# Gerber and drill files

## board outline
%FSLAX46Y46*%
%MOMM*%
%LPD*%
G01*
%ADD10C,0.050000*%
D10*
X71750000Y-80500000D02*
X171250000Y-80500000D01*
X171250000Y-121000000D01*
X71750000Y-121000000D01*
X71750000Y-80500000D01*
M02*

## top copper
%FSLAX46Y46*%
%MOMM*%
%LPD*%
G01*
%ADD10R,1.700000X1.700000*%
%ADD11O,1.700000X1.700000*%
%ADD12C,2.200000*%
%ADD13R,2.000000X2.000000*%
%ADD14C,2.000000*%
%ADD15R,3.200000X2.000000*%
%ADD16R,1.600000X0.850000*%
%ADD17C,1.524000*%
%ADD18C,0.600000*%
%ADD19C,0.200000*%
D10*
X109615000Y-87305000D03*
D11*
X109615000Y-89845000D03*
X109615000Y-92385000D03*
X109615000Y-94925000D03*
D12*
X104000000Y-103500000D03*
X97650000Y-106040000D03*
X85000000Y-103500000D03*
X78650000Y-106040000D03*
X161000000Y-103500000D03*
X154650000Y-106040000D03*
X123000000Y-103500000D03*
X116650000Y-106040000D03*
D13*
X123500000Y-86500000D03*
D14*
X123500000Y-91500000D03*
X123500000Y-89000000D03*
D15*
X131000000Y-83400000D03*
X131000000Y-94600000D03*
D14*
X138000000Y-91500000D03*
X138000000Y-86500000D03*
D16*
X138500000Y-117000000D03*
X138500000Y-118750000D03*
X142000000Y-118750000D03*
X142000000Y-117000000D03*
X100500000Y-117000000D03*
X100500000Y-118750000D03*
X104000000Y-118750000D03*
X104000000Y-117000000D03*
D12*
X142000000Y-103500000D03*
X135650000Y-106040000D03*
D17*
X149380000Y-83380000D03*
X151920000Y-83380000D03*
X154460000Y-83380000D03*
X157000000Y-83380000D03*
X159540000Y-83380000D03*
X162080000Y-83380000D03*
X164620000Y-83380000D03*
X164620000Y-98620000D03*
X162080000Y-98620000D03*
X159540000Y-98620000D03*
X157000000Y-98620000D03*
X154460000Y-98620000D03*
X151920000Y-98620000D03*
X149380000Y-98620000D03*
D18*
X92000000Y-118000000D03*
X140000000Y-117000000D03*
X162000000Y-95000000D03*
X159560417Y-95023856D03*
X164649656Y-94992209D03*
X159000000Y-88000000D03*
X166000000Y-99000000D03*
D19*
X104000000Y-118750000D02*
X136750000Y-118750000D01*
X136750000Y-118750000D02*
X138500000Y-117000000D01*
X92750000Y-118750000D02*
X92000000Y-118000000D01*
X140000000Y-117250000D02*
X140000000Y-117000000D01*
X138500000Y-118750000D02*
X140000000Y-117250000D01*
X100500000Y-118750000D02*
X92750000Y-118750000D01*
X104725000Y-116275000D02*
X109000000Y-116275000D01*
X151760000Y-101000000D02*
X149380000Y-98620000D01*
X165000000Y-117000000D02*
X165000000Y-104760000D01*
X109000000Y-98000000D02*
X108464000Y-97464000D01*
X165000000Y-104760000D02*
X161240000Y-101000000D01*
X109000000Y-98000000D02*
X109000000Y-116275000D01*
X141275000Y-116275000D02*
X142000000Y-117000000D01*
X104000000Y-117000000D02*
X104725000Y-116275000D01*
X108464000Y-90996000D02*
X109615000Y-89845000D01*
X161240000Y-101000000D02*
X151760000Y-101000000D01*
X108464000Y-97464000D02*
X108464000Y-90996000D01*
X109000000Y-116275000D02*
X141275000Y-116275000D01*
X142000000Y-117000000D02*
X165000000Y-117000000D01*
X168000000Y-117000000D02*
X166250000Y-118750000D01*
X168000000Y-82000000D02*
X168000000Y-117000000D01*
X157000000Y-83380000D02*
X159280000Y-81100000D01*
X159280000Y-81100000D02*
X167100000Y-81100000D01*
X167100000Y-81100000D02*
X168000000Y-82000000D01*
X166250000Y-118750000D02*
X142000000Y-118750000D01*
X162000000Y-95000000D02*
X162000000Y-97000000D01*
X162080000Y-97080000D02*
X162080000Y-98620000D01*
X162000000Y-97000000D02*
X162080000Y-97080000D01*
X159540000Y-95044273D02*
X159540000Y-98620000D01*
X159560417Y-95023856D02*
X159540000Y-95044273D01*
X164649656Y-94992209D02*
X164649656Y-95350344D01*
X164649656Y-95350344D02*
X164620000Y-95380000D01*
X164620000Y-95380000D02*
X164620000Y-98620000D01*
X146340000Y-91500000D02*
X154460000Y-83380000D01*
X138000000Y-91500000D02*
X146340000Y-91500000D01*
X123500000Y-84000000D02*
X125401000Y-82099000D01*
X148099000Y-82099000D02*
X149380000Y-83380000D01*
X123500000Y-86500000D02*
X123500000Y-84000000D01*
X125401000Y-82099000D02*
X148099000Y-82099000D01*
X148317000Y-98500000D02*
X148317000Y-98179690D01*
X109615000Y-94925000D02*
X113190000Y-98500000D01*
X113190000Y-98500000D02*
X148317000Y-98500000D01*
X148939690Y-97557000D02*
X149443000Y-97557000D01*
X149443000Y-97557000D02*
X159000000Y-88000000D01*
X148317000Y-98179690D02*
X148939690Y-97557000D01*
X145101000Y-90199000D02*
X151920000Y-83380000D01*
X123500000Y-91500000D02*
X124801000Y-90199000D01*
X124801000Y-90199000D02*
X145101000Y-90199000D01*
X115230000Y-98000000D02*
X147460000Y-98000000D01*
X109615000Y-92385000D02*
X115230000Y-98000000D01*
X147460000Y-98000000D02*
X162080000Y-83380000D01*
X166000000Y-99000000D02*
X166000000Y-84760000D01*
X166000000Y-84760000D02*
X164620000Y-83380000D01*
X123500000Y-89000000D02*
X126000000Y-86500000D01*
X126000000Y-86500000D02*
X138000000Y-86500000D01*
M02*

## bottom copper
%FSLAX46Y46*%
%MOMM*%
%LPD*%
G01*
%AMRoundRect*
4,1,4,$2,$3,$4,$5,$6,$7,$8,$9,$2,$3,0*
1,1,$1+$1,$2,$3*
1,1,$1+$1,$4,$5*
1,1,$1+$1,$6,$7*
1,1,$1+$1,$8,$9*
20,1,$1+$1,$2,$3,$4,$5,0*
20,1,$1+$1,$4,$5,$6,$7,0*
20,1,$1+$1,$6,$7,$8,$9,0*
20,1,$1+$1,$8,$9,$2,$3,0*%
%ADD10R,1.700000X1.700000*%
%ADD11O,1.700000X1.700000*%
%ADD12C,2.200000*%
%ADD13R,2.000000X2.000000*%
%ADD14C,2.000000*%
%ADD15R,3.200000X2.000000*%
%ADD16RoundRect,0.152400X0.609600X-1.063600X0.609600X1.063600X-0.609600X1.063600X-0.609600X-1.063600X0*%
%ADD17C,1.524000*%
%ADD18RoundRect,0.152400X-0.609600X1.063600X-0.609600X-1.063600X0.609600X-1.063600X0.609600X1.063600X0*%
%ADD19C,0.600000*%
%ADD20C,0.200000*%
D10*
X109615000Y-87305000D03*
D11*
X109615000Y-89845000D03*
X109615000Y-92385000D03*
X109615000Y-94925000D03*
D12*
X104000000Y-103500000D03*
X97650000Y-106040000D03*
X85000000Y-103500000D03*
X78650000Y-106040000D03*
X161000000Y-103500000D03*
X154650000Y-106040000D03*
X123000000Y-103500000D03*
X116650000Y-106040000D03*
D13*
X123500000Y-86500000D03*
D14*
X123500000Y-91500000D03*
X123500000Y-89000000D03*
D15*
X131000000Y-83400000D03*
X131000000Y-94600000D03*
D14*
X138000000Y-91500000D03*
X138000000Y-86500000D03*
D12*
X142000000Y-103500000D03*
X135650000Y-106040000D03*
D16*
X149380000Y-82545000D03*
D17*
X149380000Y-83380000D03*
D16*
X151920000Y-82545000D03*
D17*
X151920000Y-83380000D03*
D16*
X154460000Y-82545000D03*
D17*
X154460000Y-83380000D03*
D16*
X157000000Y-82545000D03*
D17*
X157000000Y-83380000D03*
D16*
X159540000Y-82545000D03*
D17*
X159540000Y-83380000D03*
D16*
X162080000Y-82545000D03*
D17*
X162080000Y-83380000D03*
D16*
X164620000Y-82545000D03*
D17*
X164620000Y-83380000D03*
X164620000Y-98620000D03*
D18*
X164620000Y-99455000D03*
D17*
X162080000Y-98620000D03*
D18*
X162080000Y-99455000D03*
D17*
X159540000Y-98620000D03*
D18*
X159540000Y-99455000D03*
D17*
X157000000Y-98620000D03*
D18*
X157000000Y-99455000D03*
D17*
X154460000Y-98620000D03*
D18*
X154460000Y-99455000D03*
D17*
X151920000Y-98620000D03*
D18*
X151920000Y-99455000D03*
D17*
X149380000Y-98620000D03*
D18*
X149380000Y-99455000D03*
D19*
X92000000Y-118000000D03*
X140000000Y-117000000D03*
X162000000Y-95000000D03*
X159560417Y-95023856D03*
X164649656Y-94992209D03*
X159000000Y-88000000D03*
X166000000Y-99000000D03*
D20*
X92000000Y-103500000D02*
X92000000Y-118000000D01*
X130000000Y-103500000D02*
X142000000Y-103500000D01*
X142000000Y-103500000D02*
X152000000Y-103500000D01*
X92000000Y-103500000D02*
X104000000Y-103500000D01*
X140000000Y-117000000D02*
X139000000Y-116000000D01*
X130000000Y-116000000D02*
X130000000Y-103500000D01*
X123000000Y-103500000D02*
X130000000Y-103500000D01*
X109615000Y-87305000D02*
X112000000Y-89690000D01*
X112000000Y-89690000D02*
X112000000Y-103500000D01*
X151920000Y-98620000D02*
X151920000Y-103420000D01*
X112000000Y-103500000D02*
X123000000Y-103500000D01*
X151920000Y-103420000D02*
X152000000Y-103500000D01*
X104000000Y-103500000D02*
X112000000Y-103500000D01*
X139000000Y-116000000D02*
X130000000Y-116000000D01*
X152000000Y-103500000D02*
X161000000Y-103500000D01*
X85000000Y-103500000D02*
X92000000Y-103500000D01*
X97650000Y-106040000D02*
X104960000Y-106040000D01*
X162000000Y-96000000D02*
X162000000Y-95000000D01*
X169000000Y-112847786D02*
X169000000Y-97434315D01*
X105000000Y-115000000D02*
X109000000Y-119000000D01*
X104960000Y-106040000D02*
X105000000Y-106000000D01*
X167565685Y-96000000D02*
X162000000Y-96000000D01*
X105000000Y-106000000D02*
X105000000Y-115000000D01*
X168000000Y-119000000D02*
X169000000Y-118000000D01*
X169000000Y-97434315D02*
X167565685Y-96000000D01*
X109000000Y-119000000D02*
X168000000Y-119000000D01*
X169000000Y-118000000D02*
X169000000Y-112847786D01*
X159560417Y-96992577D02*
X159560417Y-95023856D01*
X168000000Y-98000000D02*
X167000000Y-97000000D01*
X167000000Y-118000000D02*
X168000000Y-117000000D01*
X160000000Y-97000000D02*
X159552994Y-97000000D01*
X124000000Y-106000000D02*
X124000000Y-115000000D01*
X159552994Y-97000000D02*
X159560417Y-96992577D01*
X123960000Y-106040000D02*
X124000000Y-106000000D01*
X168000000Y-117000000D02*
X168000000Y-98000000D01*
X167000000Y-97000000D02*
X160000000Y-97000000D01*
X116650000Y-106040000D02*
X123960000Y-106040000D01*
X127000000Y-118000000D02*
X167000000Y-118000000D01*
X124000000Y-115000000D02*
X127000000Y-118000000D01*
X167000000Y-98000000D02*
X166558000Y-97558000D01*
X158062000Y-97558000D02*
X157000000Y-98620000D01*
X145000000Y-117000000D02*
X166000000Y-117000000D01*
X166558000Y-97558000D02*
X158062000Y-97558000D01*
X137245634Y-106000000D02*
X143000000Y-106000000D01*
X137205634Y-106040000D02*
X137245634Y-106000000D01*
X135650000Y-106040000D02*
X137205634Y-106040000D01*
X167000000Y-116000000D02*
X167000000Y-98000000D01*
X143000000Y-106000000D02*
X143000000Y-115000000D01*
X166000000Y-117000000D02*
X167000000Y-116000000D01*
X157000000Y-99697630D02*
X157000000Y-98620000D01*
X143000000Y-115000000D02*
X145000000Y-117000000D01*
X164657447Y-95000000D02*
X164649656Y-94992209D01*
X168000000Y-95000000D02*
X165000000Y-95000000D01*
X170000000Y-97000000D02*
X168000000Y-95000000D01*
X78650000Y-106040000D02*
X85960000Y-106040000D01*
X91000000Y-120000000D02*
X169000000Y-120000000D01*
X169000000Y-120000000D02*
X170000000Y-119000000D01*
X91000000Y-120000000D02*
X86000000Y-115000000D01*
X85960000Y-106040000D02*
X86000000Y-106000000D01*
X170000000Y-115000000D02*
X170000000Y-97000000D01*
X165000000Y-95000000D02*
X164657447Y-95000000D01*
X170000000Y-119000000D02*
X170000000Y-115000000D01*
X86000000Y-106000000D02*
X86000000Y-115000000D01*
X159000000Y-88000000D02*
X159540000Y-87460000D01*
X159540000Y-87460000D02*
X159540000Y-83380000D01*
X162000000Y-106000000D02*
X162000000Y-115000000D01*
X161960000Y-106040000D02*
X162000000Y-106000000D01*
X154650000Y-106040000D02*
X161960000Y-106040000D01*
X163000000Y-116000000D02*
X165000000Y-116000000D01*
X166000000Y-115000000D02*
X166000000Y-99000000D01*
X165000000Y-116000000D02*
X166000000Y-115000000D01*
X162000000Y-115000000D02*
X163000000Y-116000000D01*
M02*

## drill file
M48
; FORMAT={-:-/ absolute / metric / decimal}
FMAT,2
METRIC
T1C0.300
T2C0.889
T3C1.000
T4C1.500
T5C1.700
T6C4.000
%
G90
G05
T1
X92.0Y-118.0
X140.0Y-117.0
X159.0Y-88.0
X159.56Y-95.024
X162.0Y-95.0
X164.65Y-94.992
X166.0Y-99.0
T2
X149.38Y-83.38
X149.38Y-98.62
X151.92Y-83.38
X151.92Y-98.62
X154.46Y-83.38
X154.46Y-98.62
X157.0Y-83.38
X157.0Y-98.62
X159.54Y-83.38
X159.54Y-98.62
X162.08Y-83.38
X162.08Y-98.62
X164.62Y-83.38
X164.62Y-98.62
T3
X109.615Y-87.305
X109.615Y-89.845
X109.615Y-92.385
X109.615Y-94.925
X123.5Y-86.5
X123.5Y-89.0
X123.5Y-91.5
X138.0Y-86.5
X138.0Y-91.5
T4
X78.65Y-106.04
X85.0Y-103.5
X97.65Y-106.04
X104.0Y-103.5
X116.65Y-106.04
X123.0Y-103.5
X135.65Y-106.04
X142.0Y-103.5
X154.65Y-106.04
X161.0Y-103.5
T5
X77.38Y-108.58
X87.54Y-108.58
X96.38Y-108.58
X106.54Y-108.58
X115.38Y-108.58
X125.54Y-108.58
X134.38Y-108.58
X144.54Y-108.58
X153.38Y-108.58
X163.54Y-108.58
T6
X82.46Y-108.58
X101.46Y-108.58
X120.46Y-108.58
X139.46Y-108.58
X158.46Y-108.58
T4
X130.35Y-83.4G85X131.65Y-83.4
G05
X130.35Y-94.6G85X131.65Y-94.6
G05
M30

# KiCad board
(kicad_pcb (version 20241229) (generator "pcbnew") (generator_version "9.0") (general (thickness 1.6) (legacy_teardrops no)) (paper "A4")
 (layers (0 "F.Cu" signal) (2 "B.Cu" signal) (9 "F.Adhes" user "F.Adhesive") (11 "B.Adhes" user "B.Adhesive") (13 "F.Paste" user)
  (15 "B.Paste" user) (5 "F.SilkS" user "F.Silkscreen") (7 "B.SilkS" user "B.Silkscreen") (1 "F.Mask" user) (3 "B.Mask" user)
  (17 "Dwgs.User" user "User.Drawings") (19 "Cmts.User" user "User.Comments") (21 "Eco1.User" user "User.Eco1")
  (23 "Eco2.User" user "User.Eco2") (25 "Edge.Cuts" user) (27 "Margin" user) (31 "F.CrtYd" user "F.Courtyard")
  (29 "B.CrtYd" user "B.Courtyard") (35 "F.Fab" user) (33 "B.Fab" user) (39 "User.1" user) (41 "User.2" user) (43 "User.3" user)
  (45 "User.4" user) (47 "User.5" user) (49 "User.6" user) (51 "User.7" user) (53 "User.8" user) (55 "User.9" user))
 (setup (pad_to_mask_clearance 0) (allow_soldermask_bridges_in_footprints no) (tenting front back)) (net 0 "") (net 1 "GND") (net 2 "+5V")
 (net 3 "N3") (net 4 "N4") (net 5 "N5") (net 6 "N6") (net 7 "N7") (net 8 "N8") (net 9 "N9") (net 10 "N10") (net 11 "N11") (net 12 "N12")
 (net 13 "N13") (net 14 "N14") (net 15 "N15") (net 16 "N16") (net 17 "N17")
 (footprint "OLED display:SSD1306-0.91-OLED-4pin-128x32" (layer "F.Cu") (at 73.115 85.115)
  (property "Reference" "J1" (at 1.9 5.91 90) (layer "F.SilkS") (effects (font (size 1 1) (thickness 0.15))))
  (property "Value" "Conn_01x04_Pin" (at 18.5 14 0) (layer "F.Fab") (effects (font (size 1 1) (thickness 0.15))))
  (pad "1" thru_hole rect (at 36.5 2.19) (size 1.7 1.7) (drill 1) (layers "*.Cu" "*.Mask") (remove_unused_layers no) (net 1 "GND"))
  (pad "2" thru_hole oval (at 36.5 4.73) (size 1.7 1.7) (drill 1) (layers "*.Cu" "*.Mask") (remove_unused_layers no) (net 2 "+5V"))
  (pad "3" thru_hole oval (at 36.5 7.27) (size 1.7 1.7) (drill 1) (layers "*.Cu" "*.Mask") (remove_unused_layers no) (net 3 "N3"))
  (pad "4" thru_hole oval (at 36.5 9.81) (size 1.7 1.7) (drill 1) (layers "*.Cu" "*.Mask") (remove_unused_layers no) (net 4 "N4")))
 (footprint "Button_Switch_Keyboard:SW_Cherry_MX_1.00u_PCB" (layer "F.Cu") (at 104 103.5)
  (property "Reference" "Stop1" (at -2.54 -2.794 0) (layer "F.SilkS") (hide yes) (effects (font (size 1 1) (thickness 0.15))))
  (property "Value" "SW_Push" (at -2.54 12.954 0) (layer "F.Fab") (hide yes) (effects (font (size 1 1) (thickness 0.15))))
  (pad "" np_thru_hole circle (at -7.62 5.08) (size 1.7 1.7) (drill 1.7) (layers "*.Cu" "*.Mask"))
  (pad "" np_thru_hole circle (at -2.54 5.08) (size 4 4) (drill 4) (layers "*.Cu" "*.Mask"))
  (pad "" np_thru_hole circle (at 2.54 5.08) (size 1.7 1.7) (drill 1.7) (layers "*.Cu" "*.Mask"))
  (pad "1" thru_hole circle (at 0 0) (size 2.2 2.2) (drill 1.5) (layers "*.Cu" "*.Mask") (remove_unused_layers no) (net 1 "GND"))
  (pad "2" thru_hole circle (at -6.35 2.54) (size 2.2 2.2) (drill 1.5) (layers "*.Cu" "*.Mask") (remove_unused_layers no) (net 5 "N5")))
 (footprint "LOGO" (layer "F.Cu") (at 120 108.58)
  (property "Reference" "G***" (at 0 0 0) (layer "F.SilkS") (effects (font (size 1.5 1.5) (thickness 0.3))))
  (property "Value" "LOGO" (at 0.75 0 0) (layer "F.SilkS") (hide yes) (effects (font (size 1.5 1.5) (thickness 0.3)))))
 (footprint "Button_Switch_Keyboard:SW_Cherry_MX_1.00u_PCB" (layer "F.Cu") (at 85 103.5)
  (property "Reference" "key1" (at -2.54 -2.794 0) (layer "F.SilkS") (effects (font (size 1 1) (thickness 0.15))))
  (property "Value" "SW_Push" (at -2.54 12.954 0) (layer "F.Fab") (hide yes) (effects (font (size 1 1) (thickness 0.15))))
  (pad "" np_thru_hole circle (at -7.62 5.08) (size 1.7 1.7) (drill 1.7) (layers "*.Cu" "*.Mask"))
  (pad "" np_thru_hole circle (at -2.54 5.08) (size 4 4) (drill 4) (layers "*.Cu" "*.Mask"))
  (pad "" np_thru_hole circle (at 2.54 5.08) (size 1.7 1.7) (drill 1.7) (layers "*.Cu" "*.Mask"))
  (pad "1" thru_hole circle (at 0 0) (size 2.2 2.2) (drill 1.5) (layers "*.Cu" "*.Mask") (remove_unused_layers no) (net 1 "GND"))
  (pad "2" thru_hole circle (at -6.35 2.54) (size 2.2 2.2) (drill 1.5) (layers "*.Cu" "*.Mask") (remove_unused_layers no) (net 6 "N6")))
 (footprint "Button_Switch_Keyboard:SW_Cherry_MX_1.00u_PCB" (layer "F.Cu") (at 161 103.5)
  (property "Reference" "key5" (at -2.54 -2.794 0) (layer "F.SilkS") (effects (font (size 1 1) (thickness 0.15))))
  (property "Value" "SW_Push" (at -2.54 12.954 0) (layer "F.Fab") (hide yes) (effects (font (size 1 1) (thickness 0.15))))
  (pad "" np_thru_hole circle (at -7.62 5.08) (size 1.7 1.7) (drill 1.7) (layers "*.Cu" "*.Mask"))
  (pad "" np_thru_hole circle (at -2.54 5.08) (size 4 4) (drill 4) (layers "*.Cu" "*.Mask"))
  (pad "" np_thru_hole circle (at 2.54 5.08) (size 1.7 1.7) (drill 1.7) (layers "*.Cu" "*.Mask"))
  (pad "1" thru_hole circle (at 0 0) (size 2.2 2.2) (drill 1.5) (layers "*.Cu" "*.Mask") (remove_unused_layers no) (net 1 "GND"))
  (pad "2" thru_hole circle (at -6.35 2.54) (size 2.2 2.2) (drill 1.5) (layers "*.Cu" "*.Mask") (remove_unused_layers no) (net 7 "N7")))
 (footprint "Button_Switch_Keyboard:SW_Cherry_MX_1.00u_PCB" (layer "F.Cu") (at 123 103.5)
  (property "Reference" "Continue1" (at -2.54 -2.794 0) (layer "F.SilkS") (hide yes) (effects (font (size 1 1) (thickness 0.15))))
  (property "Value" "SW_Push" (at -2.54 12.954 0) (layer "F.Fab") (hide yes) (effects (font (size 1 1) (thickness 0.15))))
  (pad "" np_thru_hole circle (at -7.62 5.08) (size 1.7 1.7) (drill 1.7) (layers "*.Cu" "*.Mask"))
  (pad "" np_thru_hole circle (at -2.54 5.08) (size 4 4) (drill 4) (layers "*.Cu" "*.Mask"))
  (pad "" np_thru_hole circle (at 2.54 5.08) (size 1.7 1.7) (drill 1.7) (layers "*.Cu" "*.Mask"))
  (pad "1" thru_hole circle (at 0 0) (size 2.2 2.2) (drill 1.5) (layers "*.Cu" "*.Mask") (remove_unused_layers no) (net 1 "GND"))
  (pad "2" thru_hole circle (at -6.35 2.54) (size 2.2 2.2) (drill 1.5) (layers "*.Cu" "*.Mask") (remove_unused_layers no) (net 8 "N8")))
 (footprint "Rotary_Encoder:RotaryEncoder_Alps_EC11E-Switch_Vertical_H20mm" (layer "F.Cu") (at 123.5 86.5)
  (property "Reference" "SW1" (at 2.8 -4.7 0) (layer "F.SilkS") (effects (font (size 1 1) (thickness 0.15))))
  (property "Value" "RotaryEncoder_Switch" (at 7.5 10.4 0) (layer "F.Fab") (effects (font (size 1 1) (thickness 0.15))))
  (pad "A" thru_hole rect (at 0 0) (size 2 2) (drill 1) (layers "*.Cu" "*.Mask") (remove_unused_layers no) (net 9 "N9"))
  (pad "B" thru_hole circle (at 0 5) (size 2 2) (drill 1) (layers "*.Cu" "*.Mask") (remove_unused_layers no) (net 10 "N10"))
  (pad "C" thru_hole circle (at 0 2.5) (size 2 2) (drill 1) (layers "*.Cu" "*.Mask") (remove_unused_layers no) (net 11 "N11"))
  (pad "MP" thru_hole rect (at 7.5 -3.1) (size 3.2 2) (drill oval 2.8 1.5) (layers "*.Cu" "*.Mask") (remove_unused_layers no))
  (pad "MP" thru_hole rect (at 7.5 8.1) (size 3.2 2) (drill oval 2.8 1.5) (layers "*.Cu" "*.Mask") (remove_unused_layers no))
  (pad "S1" thru_hole circle (at 14.5 5) (size 2 2) (drill 1) (layers "*.Cu" "*.Mask") (remove_unused_layers no) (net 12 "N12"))
  (pad "S2" thru_hole circle (at 14.5 0) (size 2 2) (drill 1) (layers "*.Cu" "*.Mask") (remove_unused_layers no) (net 11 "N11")))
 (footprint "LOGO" (layer "F.Cu") (at 162.5 111.5)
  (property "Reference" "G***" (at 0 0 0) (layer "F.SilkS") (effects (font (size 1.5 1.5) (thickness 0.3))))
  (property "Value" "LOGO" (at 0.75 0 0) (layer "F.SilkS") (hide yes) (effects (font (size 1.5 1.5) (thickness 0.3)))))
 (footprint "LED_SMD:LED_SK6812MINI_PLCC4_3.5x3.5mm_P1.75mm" (layer "F.Cu") (at 140.25 117.875)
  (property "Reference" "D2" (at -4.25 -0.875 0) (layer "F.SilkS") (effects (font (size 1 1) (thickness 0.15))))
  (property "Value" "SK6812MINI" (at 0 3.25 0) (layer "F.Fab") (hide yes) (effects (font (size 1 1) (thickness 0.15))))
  (pad "1" smd rect (at -1.75 -0.875) (size 1.6 0.85) (layers "F.Cu" "F.Mask" "F.Paste") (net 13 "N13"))
  (pad "2" smd rect (at -1.75 0.875) (size 1.6 0.85) (layers "F.Cu" "F.Mask" "F.Paste") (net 1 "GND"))
  (pad "3" smd rect (at 1.75 0.875) (size 1.6 0.85) (layers "F.Cu" "F.Mask" "F.Paste") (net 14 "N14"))
  (pad "4" smd rect (at 1.75 -0.875) (size 1.6 0.85) (layers "F.Cu" "F.Mask" "F.Paste") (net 2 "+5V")))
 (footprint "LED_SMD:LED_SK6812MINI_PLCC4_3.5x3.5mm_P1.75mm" (layer "F.Cu") (at 102.25 117.875)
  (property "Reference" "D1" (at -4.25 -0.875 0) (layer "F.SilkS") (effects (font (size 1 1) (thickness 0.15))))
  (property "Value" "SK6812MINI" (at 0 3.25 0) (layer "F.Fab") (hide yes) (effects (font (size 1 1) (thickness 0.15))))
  (pad "1" smd rect (at -1.75 -0.875) (size 1.6 0.85) (layers "F.Cu" "F.Mask" "F.Paste") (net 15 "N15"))
  (pad "2" smd rect (at -1.75 0.875) (size 1.6 0.85) (layers "F.Cu" "F.Mask" "F.Paste") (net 1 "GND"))
  (pad "3" smd rect (at 1.75 0.875) (size 1.6 0.85) (layers "F.Cu" "F.Mask" "F.Paste") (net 13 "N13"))
  (pad "4" smd rect (at 1.75 -0.875) (size 1.6 0.85) (layers "F.Cu" "F.Mask" "F.Paste") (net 2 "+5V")))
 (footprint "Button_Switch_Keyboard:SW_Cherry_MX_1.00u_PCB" (layer "F.Cu") (at 142 103.5)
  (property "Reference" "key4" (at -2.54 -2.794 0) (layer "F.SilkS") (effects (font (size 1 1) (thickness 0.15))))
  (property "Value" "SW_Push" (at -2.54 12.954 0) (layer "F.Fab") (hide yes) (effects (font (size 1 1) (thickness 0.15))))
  (pad "" np_thru_hole circle (at -7.62 5.08) (size 1.7 1.7) (drill 1.7) (layers "*.Cu" "*.Mask"))
  (pad "" np_thru_hole circle (at -2.54 5.08) (size 4 4) (drill 4) (layers "*.Cu" "*.Mask"))
  (pad "" np_thru_hole circle (at 2.54 5.08) (size 1.7 1.7) (drill 1.7) (layers "*.Cu" "*.Mask"))
  (pad "1" thru_hole circle (at 0 0) (size 2.2 2.2) (drill 1.5) (layers "*.Cu" "*.Mask") (remove_unused_layers no) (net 1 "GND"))
  (pad "2" thru_hole circle (at -6.35 2.54) (size 2.2 2.2) (drill 1.5) (layers "*.Cu" "*.Mask") (remove_unused_layers no) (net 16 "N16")))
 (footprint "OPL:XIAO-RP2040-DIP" (layer "B.Cu") (at 157 91 -90)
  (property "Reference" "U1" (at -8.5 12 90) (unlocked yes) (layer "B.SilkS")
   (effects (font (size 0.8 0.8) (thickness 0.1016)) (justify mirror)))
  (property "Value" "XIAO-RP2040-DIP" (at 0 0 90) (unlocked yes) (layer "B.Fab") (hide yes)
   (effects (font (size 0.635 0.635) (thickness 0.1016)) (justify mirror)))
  (pad "1" smd roundrect (at -8.455 7.62 90) (size 2.432 1.524) (layers "B.Cu" "B.Mask") (roundrect_rratio 0.1) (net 9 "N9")
   (thermal_bridge_angle 45))
  (pad "1" thru_hole circle (at -7.62 7.62 90) (size 1.524 1.524) (drill 0.889) (layers "*.Cu" "*.Mask") (remove_unused_layers no)
   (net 9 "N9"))
  (pad "2" smd roundrect (at -8.455 5.08 90) (size 2.432 1.524) (layers "B.Cu" "B.Mask") (roundrect_rratio 0.1) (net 10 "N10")
   (thermal_bridge_angle 45))
  (pad "2" thru_hole circle (at -7.62 5.08 90) (size 1.524 1.524) (drill 0.889) (layers "*.Cu" "*.Mask") (remove_unused_layers no)
   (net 10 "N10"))
  (pad "3" smd roundrect (at -8.455 2.54 90) (size 2.432 1.524) (layers "B.Cu" "B.Mask") (roundrect_rratio 0.1) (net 12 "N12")
   (thermal_bridge_angle 45))
  (pad "3" thru_hole circle (at -7.62 2.54 90) (size 1.524 1.524) (drill 0.889) (layers "*.Cu" "*.Mask") (remove_unused_layers no)
   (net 12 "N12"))
  (pad "4" smd roundrect (at -8.455 0 90) (size 2.432 1.524) (layers "B.Cu" "B.Mask") (roundrect_rratio 0.1) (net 14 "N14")
   (thermal_bridge_angle 45))
  (pad "4" thru_hole circle (at -7.62 0 90) (size 1.524 1.524) (drill 0.889) (layers "*.Cu" "*.Mask") (remove_unused_layers no)
   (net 14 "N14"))
  (pad "5" smd roundrect (at -8.455 -2.54 90) (size 2.432 1.524) (layers "B.Cu" "B.Mask") (roundrect_rratio 0.1) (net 4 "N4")
   (thermal_bridge_angle 45))
  (pad "5" thru_hole circle (at -7.62 -2.54 90) (size 1.524 1.524) (drill 0.889) (layers "*.Cu" "*.Mask") (remove_unused_layers no)
   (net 4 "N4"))
  (pad "6" smd roundrect (at -8.455 -5.08 90) (size 2.432 1.524) (layers "B.Cu" "B.Mask") (roundrect_rratio 0.1) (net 3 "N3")
   (thermal_bridge_angle 45))
  (pad "6" thru_hole circle (at -7.62 -5.08 90) (size 1.524 1.524) (drill 0.889) (layers "*.Cu" "*.Mask") (remove_unused_layers no)
   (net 3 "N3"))
  (pad "7" smd roundrect (at -8.455 -7.62 90) (size 2.432 1.524) (layers "B.Cu" "B.Mask") (roundrect_rratio 0.1) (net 7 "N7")
   (thermal_bridge_angle 45))
  (pad "7" thru_hole circle (at -7.62 -7.62 90) (size 1.524 1.524) (drill 0.889) (layers "*.Cu" "*.Mask") (remove_unused_layers no)
   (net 7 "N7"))
  (pad "8" thru_hole circle (at 7.62 -7.62 270) (size 1.524 1.524) (drill 0.889) (layers "*.Cu" "*.Mask") (remove_unused_layers no)
   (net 6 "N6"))
  (pad "8" smd roundrect (at 8.455 -7.62 270) (size 2.432 1.524) (layers "B.Cu" "B.Mask") (roundrect_rratio 0.1) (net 6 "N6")
   (thermal_bridge_angle 45))
  (pad "9" thru_hole circle (at 7.62 -5.08 270) (size 1.524 1.524) (drill 0.889) (layers "*.Cu" "*.Mask") (remove_unused_layers no)
   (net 5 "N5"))
  (pad "9" smd roundrect (at 8.455 -5.08 270) (size 2.432 1.524) (layers "B.Cu" "B.Mask") (roundrect_rratio 0.1) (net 5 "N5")
   (thermal_bridge_angle 45))
  (pad "10" thru_hole circle (at 7.62 -2.54 270) (size 1.524 1.524) (drill 0.889) (layers "*.Cu" "*.Mask") (remove_unused_layers no)
   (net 8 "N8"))
  (pad "10" smd roundrect (at 8.455 -2.54 270) (size 2.432 1.524) (layers "B.Cu" "B.Mask") (roundrect_rratio 0.1) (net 8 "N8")
   (thermal_bridge_angle 45))
  (pad "11" thru_hole circle (at 7.62 0 270) (size 1.524 1.524) (drill 0.889) (layers "*.Cu" "*.Mask") (remove_unused_layers no)
   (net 16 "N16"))
  (pad "11" smd roundrect (at 8.455 0 270) (size 2.432 1.524) (layers "B.Cu" "B.Mask") (roundrect_rratio 0.1) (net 16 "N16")
   (thermal_bridge_angle 45))
  (pad "12" thru_hole circle (at 7.62 2.54 270) (size 1.524 1.524) (drill 0.889) (layers "*.Cu" "*.Mask") (remove_unused_layers no)
   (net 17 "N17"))
  (pad "12" smd roundrect (at 8.455 2.54 270) (size 2.432 1.524) (layers "B.Cu" "B.Mask") (roundrect_rratio 0.1) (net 17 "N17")
   (thermal_bridge_angle 45))
  (pad "13" thru_hole circle (at 7.62 5.08 270) (size 1.524 1.524) (drill 0.889) (layers "*.Cu" "*.Mask") (remove_unused_layers no)
   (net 1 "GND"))
  (pad "13" smd roundrect (at 8.455 5.08 270) (size 2.432 1.524) (layers "B.Cu" "B.Mask") (roundrect_rratio 0.1) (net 1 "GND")
   (thermal_bridge_angle 45))
  (pad "14" thru_hole circle (at 7.62 7.62 270) (size 1.524 1.524) (drill 0.889) (layers "*.Cu" "*.Mask") (remove_unused_layers no)
   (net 2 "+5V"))
  (pad "14" smd roundrect (at 8.455 7.62 270) (size 2.432 1.524) (layers "B.Cu" "B.Mask") (roundrect_rratio 0.1) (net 2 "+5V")
   (thermal_bridge_angle 45)))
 (gr_rect (start 71.75 80.5) (end 171.25 121) (stroke (width 0.05) (type default)) (fill no) (layer "Edge.Cuts"))
 (segment (start 104 118.75) (end 136.75 118.75) (width 0.2) (layer "F.Cu") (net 13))
 (segment (start 136.75 118.75) (end 138.5 117) (width 0.2) (layer "F.Cu") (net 13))
 (segment (start 92.75 118.75) (end 92 118) (width 0.2) (layer "F.Cu") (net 1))
 (segment (start 140 117.25) (end 140 117) (width 0.2) (layer "F.Cu") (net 1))
 (segment (start 138.5 118.75) (end 140 117.25) (width 0.2) (layer "F.Cu") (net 1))
 (segment (start 100.5 118.75) (end 92.75 118.75) (width 0.2) (layer "F.Cu") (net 1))
 (via (at 92 118) (size 0.6) (drill 0.3) (layers "F.Cu" "B.Cu") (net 1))
 (via (at 140 117) (size 0.6) (drill 0.3) (layers "F.Cu" "B.Cu") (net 1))
 (segment (start 92 103.5) (end 92 118) (width 0.2) (layer "B.Cu") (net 1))
 (segment (start 130 103.5) (end 142 103.5) (width 0.2) (layer "B.Cu") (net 1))
 (segment (start 142 103.5) (end 152 103.5) (width 0.2) (layer "B.Cu") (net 1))
 (segment (start 92 103.5) (end 104 103.5) (width 0.2) (layer "B.Cu") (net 1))
 (segment (start 140 117) (end 139 116) (width 0.2) (layer "B.Cu") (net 1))
 (segment (start 130 116) (end 130 103.5) (width 0.2) (layer "B.Cu") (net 1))
 (segment (start 123 103.5) (end 130 103.5) (width 0.2) (layer "B.Cu") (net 1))
 (segment (start 109.615 87.305) (end 112 89.69) (width 0.2) (layer "B.Cu") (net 1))
 (segment (start 112 89.69) (end 112 103.5) (width 0.2) (layer "B.Cu") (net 1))
 (segment (start 151.92 98.62) (end 151.92 103.42) (width 0.2) (layer "B.Cu") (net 1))
 (segment (start 112 103.5) (end 123 103.5) (width 0.2) (layer "B.Cu") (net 1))
 (segment (start 151.92 103.42) (end 152 103.5) (width 0.2) (layer "B.Cu") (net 1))
 (segment (start 104 103.5) (end 112 103.5) (width 0.2) (layer "B.Cu") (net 1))
 (segment (start 139 116) (end 130 116) (width 0.2) (layer "B.Cu") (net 1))
 (segment (start 152 103.5) (end 161 103.5) (width 0.2) (layer "B.Cu") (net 1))
 (segment (start 85 103.5) (end 92 103.5) (width 0.2) (layer "B.Cu") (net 1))
 (segment (start 104.725 116.275) (end 109 116.275) (width 0.2) (layer "F.Cu") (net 2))
 (segment (start 151.76 101) (end 149.38 98.62) (width 0.2) (layer "F.Cu") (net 2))
 (segment (start 165 117) (end 165 104.76) (width 0.2) (layer "F.Cu") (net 2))
 (segment (start 109 98) (end 108.464 97.464) (width 0.2) (layer "F.Cu") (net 2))
 (segment (start 165 104.76) (end 161.24 101) (width 0.2) (layer "F.Cu") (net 2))
 (segment (start 109 98) (end 109 116.275) (width 0.2) (layer "F.Cu") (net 2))
 (segment (start 141.275 116.275) (end 142 117) (width 0.2) (layer "F.Cu") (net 2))
 (segment (start 104 117) (end 104.725 116.275) (width 0.2) (layer "F.Cu") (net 2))
 (segment (start 108.464 90.996) (end 109.615 89.845) (width 0.2) (layer "F.Cu") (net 2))
 (segment (start 161.24 101) (end 151.76 101) (width 0.2) (layer "F.Cu") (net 2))
 (segment (start 108.464 97.464) (end 108.464 90.996) (width 0.2) (layer "F.Cu") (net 2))
 (segment (start 109 116.275) (end 141.275 116.275) (width 0.2) (layer "F.Cu") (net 2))
 (segment (start 142 117) (end 165 117) (width 0.2) (layer "F.Cu") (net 2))
 (segment (start 168 117) (end 166.25 118.75) (width 0.2) (layer "F.Cu") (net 14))
 (segment (start 168 82) (end 168 117) (width 0.2) (layer "F.Cu") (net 14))
 (segment (start 157 83.38) (end 159.28 81.1) (width 0.2) (layer "F.Cu") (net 14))
 (segment (start 159.28 81.1) (end 167.1 81.1) (width 0.2) (layer "F.Cu") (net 14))
 (segment (start 167.1 81.1) (end 168 82) (width 0.2) (layer "F.Cu") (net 14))
 (segment (start 166.25 118.75) (end 142 118.75) (width 0.2) (layer "F.Cu") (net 14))
 (segment (start 162 95) (end 162 97) (width 0.2) (layer "F.Cu") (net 5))
 (segment (start 162.08 97.08) (end 162.08 98.62) (width 0.2) (layer "F.Cu") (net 5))
 (segment (start 162 97) (end 162.08 97.08) (width 0.2) (layer "F.Cu") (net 5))
 (via (at 162 95) (size 0.6) (drill 0.3) (layers "F.Cu" "B.Cu") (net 5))
 (segment (start 97.65 106.04) (end 104.96 106.04) (width 0.2) (layer "B.Cu") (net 5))
 (segment (start 162 96) (end 162 95) (width 0.2) (layer "B.Cu") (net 5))
 (segment (start 169 112.847786) (end 169 97.434315) (width 0.2) (layer "B.Cu") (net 5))
 (segment (start 105 115) (end 109 119) (width 0.2) (layer "B.Cu") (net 5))
 (segment (start 104.96 106.04) (end 105 106) (width 0.2) (layer "B.Cu") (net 5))
 (segment (start 167.565685 96) (end 162 96) (width 0.2) (layer "B.Cu") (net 5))
 (segment (start 105 106) (end 105 115) (width 0.2) (layer "B.Cu") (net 5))
 (segment (start 168 119) (end 169 118) (width 0.2) (layer "B.Cu") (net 5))
 (segment (start 169 97.434315) (end 167.565685 96) (width 0.2) (layer "B.Cu") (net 5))
 (segment (start 109 119) (end 168 119) (width 0.2) (layer "B.Cu") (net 5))
 (segment (start 169 118) (end 169 112.847786) (width 0.2) (layer "B.Cu") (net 5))
 (segment (start 159.54 95.044273) (end 159.54 98.62) (width 0.2) (layer "F.Cu") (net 8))
 (segment (start 159.560417 95.023856) (end 159.54 95.044273) (width 0.2) (layer "F.Cu") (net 8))
 (via (at 159.560417 95.023856) (size 0.6) (drill 0.3) (layers "F.Cu" "B.Cu") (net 8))
 (segment (start 159.560417 96.992577) (end 159.560417 95.023856) (width 0.2) (layer "B.Cu") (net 8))
 (segment (start 168 98) (end 167 97) (width 0.2) (layer "B.Cu") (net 8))
 (segment (start 167 118) (end 168 117) (width 0.2) (layer "B.Cu") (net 8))
 (segment (start 160 97) (end 159.552994 97) (width 0.2) (layer "B.Cu") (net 8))
 (segment (start 124 106) (end 124 115) (width 0.2) (layer "B.Cu") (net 8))
 (segment (start 159.552994 97) (end 159.560417 96.992577) (width 0.2) (layer "B.Cu") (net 8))
 (segment (start 123.96 106.04) (end 124 106) (width 0.2) (layer "B.Cu") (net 8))
 (segment (start 168 117) (end 168 98) (width 0.2) (layer "B.Cu") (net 8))
 (segment (start 167 97) (end 160 97) (width 0.2) (layer "B.Cu") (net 8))
 (segment (start 116.65 106.04) (end 123.96 106.04) (width 0.2) (layer "B.Cu") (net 8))
 (segment (start 127 118) (end 167 118) (width 0.2) (layer "B.Cu") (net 8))
 (segment (start 124 115) (end 127 118) (width 0.2) (layer "B.Cu") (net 8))
 (segment (start 167 98) (end 166.558 97.558) (width 0.2) (layer "B.Cu") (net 16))
 (segment (start 158.062 97.558) (end 157 98.62) (width 0.2) (layer "B.Cu") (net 16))
 (segment (start 145 117) (end 166 117) (width 0.2) (layer "B.Cu") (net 16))
 (segment (start 166.558 97.558) (end 158.062 97.558) (width 0.2) (layer "B.Cu") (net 16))
 (segment (start 137.245634 106) (end 143 106) (width 0.2) (layer "B.Cu") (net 16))
 (segment (start 137.205634 106.04) (end 137.245634 106) (width 0.2) (layer "B.Cu") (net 16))
 (segment (start 135.65 106.04) (end 137.205634 106.04) (width 0.2) (layer "B.Cu") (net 16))
 (segment (start 167 116) (end 167 98) (width 0.2) (layer "B.Cu") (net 16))
 (segment (start 143 106) (end 143 115) (width 0.2) (layer "B.Cu") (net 16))
 (segment (start 166 117) (end 167 116) (width 0.2) (layer "B.Cu") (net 16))
 (segment (start 157 99.69763) (end 157 98.62) (width 0.2) (layer "B.Cu") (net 16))
 (segment (start 143 115) (end 145 117) (width 0.2) (layer "B.Cu") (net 16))
 (segment (start 164.649656 94.992209) (end 164.649656 95.350344) (width 0.2) (layer "F.Cu") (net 6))
 (segment (start 164.649656 95.350344) (end 164.62 95.38) (width 0.2) (layer "F.Cu") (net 6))
 (segment (start 164.62 95.38) (end 164.62 98.62) (width 0.2) (layer "F.Cu") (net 6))
 (via (at 164.649656 94.992209) (size 0.6) (drill 0.3) (layers "F.Cu" "B.Cu") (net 6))
 (segment (start 164.657447 95) (end 164.649656 94.992209) (width 0.2) (layer "B.Cu") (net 6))
 (segment (start 168 95) (end 165 95) (width 0.2) (layer "B.Cu") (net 6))
 (segment (start 170 97) (end 168 95) (width 0.2) (layer "B.Cu") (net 6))
 (segment (start 78.65 106.04) (end 85.96 106.04) (width 0.2) (layer "B.Cu") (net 6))
 (segment (start 91 120) (end 169 120) (width 0.2) (layer "B.Cu") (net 6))
 (segment (start 169 120) (end 170 119) (width 0.2) (layer "B.Cu") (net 6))
 (segment (start 91 120) (end 86 115) (width 0.2) (layer "B.Cu") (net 6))
 (segment (start 85.96 106.04) (end 86 106) (width 0.2) (layer "B.Cu") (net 6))
 (segment (start 170 115) (end 170 97) (width 0.2) (layer "B.Cu") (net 6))
 (segment (start 165 95) (end 164.657447 95) (width 0.2) (layer "B.Cu") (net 6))
 (segment (start 170 119) (end 170 115) (width 0.2) (layer "B.Cu") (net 6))
 (segment (start 86 106) (end 86 115) (width 0.2) (layer "B.Cu") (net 6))
 (segment (start 146.34 91.5) (end 154.46 83.38) (width 0.2) (layer "F.Cu") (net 12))
 (segment (start 138 91.5) (end 146.34 91.5) (width 0.2) (layer "F.Cu") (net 12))
 (segment (start 123.5 84) (end 125.401 82.099) (width 0.2) (layer "F.Cu") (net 9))
 (segment (start 148.099 82.099) (end 149.38 83.38) (width 0.2) (layer "F.Cu") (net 9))
 (segment (start 123.5 86.5) (end 123.5 84) (width 0.2) (layer "F.Cu") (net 9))
 (segment (start 125.401 82.099) (end 148.099 82.099) (width 0.2) (layer "F.Cu") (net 9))
 (segment (start 148.317 98.5) (end 148.317 98.17969) (width 0.2) (layer "F.Cu") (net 4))
 (segment (start 109.615 94.925) (end 113.19 98.5) (width 0.2) (layer "F.Cu") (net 4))
 (segment (start 113.19 98.5) (end 148.317 98.5) (width 0.2) (layer "F.Cu") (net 4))
 (segment (start 148.93969 97.557) (end 149.443 97.557) (width 0.2) (layer "F.Cu") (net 4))
 (segment (start 149.443 97.557) (end 159 88) (width 0.2) (layer "F.Cu") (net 4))
 (segment (start 148.317 98.17969) (end 148.93969 97.557) (width 0.2) (layer "F.Cu") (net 4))
 (via (at 159 88) (size 0.6) (drill 0.3) (layers "F.Cu" "B.Cu") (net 4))
 (segment (start 159 88) (end 159.54 87.46) (width 0.2) (layer "B.Cu") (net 4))
 (segment (start 159.54 87.46) (end 159.54 83.38) (width 0.2) (layer "B.Cu") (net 4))
 (segment (start 145.101 90.199) (end 151.92 83.38) (width 0.2) (layer "F.Cu") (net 10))
 (segment (start 123.5 91.5) (end 124.801 90.199) (width 0.2) (layer "F.Cu") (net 10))
 (segment (start 124.801 90.199) (end 145.101 90.199) (width 0.2) (layer "F.Cu") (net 10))
 (segment (start 115.23 98) (end 147.46 98) (width 0.2) (layer "F.Cu") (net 3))
 (segment (start 109.615 92.385) (end 115.23 98) (width 0.2) (layer "F.Cu") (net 3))
 (segment (start 147.46 98) (end 162.08 83.38) (width 0.2) (layer "F.Cu") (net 3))
 (segment (start 166 99) (end 166 84.76) (width 0.2) (layer "F.Cu") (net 7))
 (segment (start 166 84.76) (end 164.62 83.38) (width 0.2) (layer "F.Cu") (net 7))
 (via (at 166 99) (size 0.6) (drill 0.3) (layers "F.Cu" "B.Cu") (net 7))
 (segment (start 162 106) (end 162 115) (width 0.2) (layer "B.Cu") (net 7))
 (segment (start 161.96 106.04) (end 162 106) (width 0.2) (layer "B.Cu") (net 7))
 (segment (start 154.65 106.04) (end 161.96 106.04) (width 0.2) (layer "B.Cu") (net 7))
 (segment (start 163 116) (end 165 116) (width 0.2) (layer "B.Cu") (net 7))
 (segment (start 166 115) (end 166 99) (width 0.2) (layer "B.Cu") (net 7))
 (segment (start 165 116) (end 166 115) (width 0.2) (layer "B.Cu") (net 7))
 (segment (start 162 115) (end 163 116) (width 0.2) (layer "B.Cu") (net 7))
 (segment (start 123.5 89) (end 126 86.5) (width 0.2) (layer "F.Cu") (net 11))
 (segment (start 126 86.5) (end 138 86.5) (width 0.2) (layer "F.Cu") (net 11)))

